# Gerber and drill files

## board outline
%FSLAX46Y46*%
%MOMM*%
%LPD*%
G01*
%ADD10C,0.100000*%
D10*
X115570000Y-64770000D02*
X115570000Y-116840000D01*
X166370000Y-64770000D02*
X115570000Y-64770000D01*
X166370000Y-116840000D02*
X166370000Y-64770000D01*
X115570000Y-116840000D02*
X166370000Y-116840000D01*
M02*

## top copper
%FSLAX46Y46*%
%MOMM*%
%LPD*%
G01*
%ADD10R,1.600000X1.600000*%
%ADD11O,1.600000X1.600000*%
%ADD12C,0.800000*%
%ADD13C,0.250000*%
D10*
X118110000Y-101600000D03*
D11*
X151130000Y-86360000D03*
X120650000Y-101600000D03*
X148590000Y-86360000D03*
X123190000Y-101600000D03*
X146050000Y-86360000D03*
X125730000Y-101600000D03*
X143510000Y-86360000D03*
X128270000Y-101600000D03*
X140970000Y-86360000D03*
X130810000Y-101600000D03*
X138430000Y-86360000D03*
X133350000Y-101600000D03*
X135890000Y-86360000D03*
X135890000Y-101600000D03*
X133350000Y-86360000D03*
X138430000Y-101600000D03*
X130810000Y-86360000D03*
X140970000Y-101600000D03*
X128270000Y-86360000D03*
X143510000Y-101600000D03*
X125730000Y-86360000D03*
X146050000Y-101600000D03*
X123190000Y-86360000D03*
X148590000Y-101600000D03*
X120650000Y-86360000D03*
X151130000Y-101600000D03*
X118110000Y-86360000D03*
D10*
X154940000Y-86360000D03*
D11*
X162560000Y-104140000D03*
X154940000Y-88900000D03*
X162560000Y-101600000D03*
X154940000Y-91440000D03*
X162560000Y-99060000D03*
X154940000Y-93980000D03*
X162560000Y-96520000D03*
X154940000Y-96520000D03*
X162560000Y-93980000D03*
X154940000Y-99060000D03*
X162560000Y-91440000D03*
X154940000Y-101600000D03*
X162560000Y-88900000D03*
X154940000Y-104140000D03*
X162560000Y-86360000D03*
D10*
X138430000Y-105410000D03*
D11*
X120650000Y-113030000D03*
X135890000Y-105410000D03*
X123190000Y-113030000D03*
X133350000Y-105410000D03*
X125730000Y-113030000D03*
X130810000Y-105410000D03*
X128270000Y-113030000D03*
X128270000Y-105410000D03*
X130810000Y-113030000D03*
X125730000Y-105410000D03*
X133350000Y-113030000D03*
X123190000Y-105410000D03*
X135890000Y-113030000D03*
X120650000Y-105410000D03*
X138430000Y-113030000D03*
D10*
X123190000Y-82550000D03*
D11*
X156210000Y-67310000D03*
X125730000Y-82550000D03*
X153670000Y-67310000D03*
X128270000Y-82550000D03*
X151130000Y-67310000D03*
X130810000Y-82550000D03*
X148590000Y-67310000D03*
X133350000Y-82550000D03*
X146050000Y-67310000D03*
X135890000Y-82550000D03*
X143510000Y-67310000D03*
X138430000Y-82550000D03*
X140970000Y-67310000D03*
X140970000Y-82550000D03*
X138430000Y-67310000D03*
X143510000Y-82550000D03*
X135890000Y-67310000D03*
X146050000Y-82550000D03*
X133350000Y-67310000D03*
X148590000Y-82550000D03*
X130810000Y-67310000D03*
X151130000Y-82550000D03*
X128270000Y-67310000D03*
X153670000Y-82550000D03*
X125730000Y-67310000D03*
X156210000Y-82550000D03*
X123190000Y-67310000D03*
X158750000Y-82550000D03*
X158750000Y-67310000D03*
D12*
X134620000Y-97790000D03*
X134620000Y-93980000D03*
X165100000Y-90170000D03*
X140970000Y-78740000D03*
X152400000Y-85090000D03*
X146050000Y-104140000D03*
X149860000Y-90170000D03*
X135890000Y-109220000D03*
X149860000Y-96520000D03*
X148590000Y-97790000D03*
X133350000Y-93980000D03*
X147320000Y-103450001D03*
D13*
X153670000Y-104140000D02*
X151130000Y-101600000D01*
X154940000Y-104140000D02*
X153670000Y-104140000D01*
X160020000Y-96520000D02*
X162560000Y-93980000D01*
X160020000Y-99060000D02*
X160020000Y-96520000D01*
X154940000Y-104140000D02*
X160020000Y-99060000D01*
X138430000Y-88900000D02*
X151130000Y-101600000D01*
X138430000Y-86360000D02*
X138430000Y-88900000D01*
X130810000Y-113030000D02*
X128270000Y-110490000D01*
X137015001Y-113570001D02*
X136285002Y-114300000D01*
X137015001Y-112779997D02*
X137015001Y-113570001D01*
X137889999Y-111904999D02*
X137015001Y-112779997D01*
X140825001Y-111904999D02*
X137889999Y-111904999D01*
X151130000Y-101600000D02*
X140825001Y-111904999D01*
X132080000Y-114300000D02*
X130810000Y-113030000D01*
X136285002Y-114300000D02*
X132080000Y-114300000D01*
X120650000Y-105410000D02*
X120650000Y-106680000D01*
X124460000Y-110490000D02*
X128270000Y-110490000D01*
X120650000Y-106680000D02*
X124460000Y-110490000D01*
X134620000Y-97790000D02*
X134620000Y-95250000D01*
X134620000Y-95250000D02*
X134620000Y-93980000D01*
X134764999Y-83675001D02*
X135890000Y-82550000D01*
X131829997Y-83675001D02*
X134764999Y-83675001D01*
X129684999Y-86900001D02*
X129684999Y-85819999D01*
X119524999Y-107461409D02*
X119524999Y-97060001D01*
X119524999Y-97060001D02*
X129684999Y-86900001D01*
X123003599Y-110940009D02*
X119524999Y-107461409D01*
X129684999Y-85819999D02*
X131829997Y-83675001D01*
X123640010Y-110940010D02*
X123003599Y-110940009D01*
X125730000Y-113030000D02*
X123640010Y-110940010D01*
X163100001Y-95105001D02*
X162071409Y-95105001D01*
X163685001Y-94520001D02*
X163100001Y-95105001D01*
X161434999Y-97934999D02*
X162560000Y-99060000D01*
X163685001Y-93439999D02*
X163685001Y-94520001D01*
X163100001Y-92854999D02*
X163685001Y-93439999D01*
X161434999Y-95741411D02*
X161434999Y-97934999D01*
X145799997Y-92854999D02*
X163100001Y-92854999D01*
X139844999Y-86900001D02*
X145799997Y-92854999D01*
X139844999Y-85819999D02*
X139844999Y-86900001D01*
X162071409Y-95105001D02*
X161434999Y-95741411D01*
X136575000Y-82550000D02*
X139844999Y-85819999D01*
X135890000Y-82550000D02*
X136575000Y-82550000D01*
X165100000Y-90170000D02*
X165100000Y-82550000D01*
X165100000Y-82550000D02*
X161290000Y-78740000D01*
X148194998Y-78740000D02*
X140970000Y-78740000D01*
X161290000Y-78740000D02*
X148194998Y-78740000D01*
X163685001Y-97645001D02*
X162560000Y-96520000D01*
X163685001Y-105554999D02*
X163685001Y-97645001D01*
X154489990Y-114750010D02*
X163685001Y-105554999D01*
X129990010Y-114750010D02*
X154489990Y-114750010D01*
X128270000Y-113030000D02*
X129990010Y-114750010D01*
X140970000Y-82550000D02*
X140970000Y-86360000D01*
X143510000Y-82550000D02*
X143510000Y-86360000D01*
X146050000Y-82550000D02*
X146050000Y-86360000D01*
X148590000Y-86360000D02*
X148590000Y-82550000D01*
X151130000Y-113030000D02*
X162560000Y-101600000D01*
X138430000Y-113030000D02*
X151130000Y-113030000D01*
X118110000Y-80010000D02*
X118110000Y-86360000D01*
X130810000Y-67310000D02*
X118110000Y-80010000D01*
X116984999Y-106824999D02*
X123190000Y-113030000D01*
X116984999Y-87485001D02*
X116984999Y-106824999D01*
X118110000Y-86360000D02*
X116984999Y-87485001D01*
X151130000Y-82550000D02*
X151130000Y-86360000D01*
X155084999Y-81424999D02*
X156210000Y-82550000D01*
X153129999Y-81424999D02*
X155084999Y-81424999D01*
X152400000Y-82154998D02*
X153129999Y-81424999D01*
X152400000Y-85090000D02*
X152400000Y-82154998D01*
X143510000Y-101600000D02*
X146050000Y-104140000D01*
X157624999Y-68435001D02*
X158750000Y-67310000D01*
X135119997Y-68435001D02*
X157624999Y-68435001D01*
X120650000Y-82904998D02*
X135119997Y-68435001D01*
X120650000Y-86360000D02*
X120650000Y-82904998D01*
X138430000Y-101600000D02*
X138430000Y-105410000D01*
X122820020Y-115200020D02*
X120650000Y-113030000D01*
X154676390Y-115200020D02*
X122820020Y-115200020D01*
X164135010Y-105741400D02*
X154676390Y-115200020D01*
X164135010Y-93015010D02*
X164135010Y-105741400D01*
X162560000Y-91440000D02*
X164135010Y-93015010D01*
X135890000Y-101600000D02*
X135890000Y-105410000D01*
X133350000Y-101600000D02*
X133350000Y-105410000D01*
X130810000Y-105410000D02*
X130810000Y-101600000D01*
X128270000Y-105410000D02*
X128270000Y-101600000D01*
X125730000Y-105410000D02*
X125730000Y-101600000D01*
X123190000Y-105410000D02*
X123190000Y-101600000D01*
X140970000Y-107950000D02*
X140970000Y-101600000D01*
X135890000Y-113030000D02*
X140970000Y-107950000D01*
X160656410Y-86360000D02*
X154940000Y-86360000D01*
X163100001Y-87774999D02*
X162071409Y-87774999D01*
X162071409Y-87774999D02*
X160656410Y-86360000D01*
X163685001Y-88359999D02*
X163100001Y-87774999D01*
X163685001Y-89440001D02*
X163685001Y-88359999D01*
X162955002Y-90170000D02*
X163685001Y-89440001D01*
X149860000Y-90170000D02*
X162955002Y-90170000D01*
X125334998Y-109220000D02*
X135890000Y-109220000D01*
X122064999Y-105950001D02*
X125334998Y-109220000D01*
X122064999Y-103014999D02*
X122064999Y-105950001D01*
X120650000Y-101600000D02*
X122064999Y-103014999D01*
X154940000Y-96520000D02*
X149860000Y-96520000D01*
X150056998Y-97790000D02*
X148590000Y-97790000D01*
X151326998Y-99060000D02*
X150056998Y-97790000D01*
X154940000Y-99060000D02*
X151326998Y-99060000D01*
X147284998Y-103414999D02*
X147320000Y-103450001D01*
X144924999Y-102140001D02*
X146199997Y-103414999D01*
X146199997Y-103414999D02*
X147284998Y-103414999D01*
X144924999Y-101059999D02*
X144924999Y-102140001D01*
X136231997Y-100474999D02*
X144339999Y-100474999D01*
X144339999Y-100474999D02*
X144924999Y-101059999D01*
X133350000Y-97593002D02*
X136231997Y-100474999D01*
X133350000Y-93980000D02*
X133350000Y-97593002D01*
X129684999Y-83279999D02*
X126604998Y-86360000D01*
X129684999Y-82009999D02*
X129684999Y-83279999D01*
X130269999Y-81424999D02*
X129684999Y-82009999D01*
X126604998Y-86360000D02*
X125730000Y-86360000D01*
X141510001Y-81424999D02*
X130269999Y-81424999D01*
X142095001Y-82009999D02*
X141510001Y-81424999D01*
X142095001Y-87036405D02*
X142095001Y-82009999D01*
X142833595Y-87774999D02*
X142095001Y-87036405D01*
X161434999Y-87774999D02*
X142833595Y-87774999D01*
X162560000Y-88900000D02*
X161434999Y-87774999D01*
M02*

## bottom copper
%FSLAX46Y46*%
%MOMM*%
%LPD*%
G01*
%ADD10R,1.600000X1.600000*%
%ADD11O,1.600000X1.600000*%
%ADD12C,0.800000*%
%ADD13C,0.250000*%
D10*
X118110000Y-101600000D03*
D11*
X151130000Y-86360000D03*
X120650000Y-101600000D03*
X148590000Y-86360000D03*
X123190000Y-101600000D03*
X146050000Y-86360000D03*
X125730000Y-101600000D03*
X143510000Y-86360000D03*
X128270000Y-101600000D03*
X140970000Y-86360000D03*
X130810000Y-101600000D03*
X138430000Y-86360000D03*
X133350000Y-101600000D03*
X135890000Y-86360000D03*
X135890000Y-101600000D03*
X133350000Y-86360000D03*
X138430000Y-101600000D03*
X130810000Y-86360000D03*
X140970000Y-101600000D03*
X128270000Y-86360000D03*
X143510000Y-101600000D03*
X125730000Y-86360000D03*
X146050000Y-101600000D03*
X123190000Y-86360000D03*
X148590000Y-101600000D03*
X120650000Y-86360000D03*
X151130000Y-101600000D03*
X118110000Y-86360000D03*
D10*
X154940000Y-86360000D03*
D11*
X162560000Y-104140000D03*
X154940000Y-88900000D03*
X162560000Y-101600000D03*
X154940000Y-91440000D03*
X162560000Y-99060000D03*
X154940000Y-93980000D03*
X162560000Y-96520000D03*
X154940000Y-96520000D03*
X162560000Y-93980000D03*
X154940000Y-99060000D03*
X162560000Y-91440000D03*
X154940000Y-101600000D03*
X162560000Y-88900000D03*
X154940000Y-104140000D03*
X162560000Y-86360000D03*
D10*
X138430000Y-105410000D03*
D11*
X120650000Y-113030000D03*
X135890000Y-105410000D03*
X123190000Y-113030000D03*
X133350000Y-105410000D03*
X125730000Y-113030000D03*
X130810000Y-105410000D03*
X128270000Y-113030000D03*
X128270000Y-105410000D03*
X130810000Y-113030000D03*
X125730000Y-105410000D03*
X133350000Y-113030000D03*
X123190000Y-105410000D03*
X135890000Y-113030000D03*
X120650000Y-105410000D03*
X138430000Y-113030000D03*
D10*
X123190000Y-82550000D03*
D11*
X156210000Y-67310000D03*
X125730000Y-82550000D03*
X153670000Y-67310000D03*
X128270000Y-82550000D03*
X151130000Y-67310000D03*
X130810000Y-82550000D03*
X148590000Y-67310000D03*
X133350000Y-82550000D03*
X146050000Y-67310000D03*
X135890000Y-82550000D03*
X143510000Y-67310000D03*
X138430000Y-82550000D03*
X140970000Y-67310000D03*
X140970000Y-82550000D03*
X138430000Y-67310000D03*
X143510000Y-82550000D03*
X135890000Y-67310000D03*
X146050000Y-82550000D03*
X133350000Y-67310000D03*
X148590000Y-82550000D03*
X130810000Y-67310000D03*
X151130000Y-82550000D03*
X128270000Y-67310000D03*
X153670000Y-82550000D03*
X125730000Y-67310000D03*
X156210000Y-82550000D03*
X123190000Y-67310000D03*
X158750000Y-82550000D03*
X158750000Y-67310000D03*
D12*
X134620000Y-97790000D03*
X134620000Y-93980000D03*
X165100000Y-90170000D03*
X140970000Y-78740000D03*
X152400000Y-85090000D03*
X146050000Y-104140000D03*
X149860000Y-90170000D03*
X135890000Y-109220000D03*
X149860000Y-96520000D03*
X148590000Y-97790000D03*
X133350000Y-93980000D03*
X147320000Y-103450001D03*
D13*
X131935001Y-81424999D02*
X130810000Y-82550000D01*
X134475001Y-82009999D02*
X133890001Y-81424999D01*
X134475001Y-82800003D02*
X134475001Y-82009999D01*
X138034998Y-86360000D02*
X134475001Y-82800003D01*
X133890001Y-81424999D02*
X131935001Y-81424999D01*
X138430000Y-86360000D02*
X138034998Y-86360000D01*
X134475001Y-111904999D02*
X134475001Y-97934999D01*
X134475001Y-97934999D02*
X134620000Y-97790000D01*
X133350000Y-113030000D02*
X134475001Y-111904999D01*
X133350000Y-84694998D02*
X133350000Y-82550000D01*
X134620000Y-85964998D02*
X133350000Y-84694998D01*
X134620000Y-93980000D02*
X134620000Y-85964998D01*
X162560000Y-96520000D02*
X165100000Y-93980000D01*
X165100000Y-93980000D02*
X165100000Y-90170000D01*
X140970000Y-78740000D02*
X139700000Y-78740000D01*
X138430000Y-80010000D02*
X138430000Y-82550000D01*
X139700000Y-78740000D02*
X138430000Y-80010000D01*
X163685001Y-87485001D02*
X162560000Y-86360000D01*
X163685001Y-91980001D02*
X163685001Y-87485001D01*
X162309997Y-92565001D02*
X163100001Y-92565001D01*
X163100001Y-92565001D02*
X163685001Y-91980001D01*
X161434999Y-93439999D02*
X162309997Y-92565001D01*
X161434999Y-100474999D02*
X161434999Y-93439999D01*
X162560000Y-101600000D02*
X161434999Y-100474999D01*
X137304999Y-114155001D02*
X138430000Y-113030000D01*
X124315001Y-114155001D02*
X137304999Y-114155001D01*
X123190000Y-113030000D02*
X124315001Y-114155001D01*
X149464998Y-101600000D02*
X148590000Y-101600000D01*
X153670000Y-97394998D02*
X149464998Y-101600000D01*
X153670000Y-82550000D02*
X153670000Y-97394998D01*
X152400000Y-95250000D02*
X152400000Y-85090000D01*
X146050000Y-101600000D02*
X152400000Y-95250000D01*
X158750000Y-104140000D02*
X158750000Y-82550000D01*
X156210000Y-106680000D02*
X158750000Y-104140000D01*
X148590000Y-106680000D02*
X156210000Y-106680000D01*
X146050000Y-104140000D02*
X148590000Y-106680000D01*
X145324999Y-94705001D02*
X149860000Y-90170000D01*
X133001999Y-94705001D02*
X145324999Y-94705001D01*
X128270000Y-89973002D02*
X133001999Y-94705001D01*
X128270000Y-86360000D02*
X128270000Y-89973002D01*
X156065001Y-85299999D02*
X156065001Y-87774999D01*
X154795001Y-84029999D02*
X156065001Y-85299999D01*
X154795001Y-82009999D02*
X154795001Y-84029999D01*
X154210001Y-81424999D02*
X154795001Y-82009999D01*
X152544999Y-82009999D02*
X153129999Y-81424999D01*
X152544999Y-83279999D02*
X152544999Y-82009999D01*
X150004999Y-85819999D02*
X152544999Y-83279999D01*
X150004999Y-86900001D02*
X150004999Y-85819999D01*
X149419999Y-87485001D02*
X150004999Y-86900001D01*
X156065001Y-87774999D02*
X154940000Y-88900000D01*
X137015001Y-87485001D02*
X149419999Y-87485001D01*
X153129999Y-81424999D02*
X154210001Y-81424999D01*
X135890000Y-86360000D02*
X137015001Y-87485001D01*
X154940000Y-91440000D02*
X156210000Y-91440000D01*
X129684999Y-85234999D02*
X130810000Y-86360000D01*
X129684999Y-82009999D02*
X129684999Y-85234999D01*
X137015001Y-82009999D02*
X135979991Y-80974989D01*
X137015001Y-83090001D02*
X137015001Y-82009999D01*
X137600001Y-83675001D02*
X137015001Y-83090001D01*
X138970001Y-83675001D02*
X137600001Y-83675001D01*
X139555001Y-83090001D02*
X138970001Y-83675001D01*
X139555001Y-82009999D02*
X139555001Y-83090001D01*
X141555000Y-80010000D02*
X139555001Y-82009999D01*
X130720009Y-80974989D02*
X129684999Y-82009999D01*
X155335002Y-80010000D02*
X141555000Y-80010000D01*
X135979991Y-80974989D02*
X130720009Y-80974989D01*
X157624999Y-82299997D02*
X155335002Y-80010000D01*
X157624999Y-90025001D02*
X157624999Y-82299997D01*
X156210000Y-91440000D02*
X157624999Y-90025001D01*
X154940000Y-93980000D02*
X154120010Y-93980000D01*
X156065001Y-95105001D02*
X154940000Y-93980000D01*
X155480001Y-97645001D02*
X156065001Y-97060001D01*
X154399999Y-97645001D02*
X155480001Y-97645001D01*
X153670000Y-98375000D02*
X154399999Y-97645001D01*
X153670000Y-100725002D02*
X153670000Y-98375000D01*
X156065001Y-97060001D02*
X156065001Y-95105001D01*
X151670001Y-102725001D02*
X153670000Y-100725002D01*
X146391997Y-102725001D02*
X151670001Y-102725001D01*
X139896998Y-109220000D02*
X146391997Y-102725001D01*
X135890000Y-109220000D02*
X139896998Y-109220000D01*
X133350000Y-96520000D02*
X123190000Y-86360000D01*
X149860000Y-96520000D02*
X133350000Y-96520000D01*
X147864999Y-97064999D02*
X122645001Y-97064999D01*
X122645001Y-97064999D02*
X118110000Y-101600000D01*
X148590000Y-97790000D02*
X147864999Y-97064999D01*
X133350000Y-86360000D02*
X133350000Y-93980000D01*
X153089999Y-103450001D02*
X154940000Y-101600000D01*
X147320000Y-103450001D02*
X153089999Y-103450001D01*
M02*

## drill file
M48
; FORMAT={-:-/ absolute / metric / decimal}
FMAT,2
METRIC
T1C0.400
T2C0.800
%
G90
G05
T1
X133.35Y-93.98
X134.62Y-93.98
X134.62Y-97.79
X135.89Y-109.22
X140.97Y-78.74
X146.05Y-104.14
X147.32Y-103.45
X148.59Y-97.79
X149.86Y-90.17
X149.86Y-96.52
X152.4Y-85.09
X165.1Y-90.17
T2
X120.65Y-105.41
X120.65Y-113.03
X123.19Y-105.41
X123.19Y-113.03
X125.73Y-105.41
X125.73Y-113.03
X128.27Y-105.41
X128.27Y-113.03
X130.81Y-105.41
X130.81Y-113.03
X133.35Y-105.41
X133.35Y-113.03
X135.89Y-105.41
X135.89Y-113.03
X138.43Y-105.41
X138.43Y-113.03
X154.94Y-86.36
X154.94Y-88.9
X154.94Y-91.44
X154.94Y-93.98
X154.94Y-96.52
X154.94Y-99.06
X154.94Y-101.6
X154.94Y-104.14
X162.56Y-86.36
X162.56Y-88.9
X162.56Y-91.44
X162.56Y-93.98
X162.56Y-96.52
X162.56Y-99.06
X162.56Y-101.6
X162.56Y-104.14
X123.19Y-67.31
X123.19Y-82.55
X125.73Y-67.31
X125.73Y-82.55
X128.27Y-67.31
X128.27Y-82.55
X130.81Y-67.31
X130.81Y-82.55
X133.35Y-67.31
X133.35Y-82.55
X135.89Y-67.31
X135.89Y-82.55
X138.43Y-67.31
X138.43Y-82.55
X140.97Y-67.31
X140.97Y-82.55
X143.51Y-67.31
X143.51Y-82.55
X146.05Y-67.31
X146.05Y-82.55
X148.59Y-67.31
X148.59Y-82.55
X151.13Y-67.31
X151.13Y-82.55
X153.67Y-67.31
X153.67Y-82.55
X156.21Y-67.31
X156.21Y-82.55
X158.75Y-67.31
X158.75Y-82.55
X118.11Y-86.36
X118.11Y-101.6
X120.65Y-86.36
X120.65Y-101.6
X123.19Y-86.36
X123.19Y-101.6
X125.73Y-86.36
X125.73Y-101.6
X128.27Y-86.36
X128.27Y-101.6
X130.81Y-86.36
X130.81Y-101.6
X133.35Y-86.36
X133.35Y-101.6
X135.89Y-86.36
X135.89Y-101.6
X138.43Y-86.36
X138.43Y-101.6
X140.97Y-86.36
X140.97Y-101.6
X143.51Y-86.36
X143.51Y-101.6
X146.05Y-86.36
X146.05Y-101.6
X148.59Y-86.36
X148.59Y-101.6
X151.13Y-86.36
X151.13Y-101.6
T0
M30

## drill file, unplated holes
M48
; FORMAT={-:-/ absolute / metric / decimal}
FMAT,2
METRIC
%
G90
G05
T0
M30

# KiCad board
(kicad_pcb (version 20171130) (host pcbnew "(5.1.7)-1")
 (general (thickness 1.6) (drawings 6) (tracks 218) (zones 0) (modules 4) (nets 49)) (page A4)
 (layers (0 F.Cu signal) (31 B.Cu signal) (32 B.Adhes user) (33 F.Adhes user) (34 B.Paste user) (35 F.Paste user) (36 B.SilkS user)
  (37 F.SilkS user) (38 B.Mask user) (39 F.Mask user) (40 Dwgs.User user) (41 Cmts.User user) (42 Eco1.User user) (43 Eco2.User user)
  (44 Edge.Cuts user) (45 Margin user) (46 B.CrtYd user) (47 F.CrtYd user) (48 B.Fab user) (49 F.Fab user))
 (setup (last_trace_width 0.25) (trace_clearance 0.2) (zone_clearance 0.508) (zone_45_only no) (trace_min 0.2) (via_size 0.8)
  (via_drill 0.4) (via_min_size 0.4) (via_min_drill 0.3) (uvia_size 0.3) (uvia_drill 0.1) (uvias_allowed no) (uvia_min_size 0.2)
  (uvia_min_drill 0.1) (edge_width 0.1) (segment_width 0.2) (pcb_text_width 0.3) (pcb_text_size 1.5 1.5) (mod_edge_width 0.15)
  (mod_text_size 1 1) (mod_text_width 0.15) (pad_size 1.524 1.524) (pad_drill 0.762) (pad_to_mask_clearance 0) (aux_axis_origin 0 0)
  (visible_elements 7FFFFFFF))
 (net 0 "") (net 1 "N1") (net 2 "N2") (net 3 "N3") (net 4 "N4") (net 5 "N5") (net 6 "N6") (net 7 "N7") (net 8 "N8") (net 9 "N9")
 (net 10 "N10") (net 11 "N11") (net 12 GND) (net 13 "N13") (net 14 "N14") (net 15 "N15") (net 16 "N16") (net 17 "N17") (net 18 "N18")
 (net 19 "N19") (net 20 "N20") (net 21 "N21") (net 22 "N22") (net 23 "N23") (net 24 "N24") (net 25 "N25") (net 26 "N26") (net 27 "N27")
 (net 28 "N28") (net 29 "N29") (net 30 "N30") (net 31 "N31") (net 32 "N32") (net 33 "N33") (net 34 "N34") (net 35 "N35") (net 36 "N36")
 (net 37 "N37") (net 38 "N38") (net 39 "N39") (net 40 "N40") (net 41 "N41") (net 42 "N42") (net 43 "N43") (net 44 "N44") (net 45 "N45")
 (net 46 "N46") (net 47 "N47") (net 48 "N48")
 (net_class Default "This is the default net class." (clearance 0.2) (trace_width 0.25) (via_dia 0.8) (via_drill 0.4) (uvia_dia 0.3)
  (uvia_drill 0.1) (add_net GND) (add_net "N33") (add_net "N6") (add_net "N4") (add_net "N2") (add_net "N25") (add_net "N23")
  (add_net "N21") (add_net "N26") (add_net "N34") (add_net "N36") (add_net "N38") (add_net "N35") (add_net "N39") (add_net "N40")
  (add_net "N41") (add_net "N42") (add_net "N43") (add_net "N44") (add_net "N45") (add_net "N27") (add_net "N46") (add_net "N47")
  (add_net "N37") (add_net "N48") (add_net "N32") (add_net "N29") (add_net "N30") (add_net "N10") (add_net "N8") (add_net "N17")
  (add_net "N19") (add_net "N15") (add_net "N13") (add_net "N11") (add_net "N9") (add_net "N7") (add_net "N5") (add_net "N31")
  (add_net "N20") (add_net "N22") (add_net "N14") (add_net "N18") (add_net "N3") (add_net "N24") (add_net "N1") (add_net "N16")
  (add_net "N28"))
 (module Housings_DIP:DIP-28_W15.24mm (layer F.Cu) (at 118.11 101.6 90)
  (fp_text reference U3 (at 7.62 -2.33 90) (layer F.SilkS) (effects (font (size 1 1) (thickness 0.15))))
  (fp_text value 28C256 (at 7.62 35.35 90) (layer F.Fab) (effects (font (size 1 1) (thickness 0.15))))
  (pad 1 thru_hole rect (at 0 0 90) (size 1.6 1.6) (drill 0.8) (layers *.Cu *.Mask) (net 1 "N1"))
  (pad 15 thru_hole oval (at 15.24 33.02 90) (size 1.6 1.6) (drill 0.8) (layers *.Cu *.Mask) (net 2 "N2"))
  (pad 2 thru_hole oval (at 0 2.54 90) (size 1.6 1.6) (drill 0.8) (layers *.Cu *.Mask) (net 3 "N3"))
  (pad 16 thru_hole oval (at 15.24 30.48 90) (size 1.6 1.6) (drill 0.8) (layers *.Cu *.Mask) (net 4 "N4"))
  (pad 3 thru_hole oval (at 0 5.08 90) (size 1.6 1.6) (drill 0.8) (layers *.Cu *.Mask) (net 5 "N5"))
  (pad 17 thru_hole oval (at 15.24 27.94 90) (size 1.6 1.6) (drill 0.8) (layers *.Cu *.Mask) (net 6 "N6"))
  (pad 4 thru_hole oval (at 0 7.62 90) (size 1.6 1.6) (drill 0.8) (layers *.Cu *.Mask) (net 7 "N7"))
  (pad 18 thru_hole oval (at 15.24 25.4 90) (size 1.6 1.6) (drill 0.8) (layers *.Cu *.Mask) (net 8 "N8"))
  (pad 5 thru_hole oval (at 0 10.16 90) (size 1.6 1.6) (drill 0.8) (layers *.Cu *.Mask) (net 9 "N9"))
  (pad 19 thru_hole oval (at 15.24 22.86 90) (size 1.6 1.6) (drill 0.8) (layers *.Cu *.Mask) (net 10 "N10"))
  (pad 6 thru_hole oval (at 0 12.7 90) (size 1.6 1.6) (drill 0.8) (layers *.Cu *.Mask) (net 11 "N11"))
  (pad 20 thru_hole oval (at 15.24 20.32 90) (size 1.6 1.6) (drill 0.8) (layers *.Cu *.Mask) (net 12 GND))
  (pad 7 thru_hole oval (at 0 15.24 90) (size 1.6 1.6) (drill 0.8) (layers *.Cu *.Mask) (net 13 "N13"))
  (pad 21 thru_hole oval (at 15.24 17.78 90) (size 1.6 1.6) (drill 0.8) (layers *.Cu *.Mask) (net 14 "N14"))
  (pad 8 thru_hole oval (at 0 17.78 90) (size 1.6 1.6) (drill 0.8) (layers *.Cu *.Mask) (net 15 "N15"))
  (pad 22 thru_hole oval (at 15.24 15.24 90) (size 1.6 1.6) (drill 0.8) (layers *.Cu *.Mask) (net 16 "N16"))
  (pad 9 thru_hole oval (at 0 20.32 90) (size 1.6 1.6) (drill 0.8) (layers *.Cu *.Mask) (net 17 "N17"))
  (pad 23 thru_hole oval (at 15.24 12.7 90) (size 1.6 1.6) (drill 0.8) (layers *.Cu *.Mask) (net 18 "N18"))
  (pad 10 thru_hole oval (at 0 22.86 90) (size 1.6 1.6) (drill 0.8) (layers *.Cu *.Mask) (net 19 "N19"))
  (pad 24 thru_hole oval (at 15.24 10.16 90) (size 1.6 1.6) (drill 0.8) (layers *.Cu *.Mask) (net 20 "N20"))
  (pad 11 thru_hole oval (at 0 25.4 90) (size 1.6 1.6) (drill 0.8) (layers *.Cu *.Mask) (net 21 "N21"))
  (pad 25 thru_hole oval (at 15.24 7.62 90) (size 1.6 1.6) (drill 0.8) (layers *.Cu *.Mask) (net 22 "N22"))
  (pad 12 thru_hole oval (at 0 27.94 90) (size 1.6 1.6) (drill 0.8) (layers *.Cu *.Mask) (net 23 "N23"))
  (pad 26 thru_hole oval (at 15.24 5.08 90) (size 1.6 1.6) (drill 0.8) (layers *.Cu *.Mask) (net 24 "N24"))
  (pad 13 thru_hole oval (at 0 30.48 90) (size 1.6 1.6) (drill 0.8) (layers *.Cu *.Mask) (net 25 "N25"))
  (pad 27 thru_hole oval (at 15.24 2.54 90) (size 1.6 1.6) (drill 0.8) (layers *.Cu *.Mask) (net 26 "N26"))
  (pad 14 thru_hole oval (at 0 33.02 90) (size 1.6 1.6) (drill 0.8) (layers *.Cu *.Mask) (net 12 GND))
  (pad 28 thru_hole oval (at 15.24 0 90) (size 1.6 1.6) (drill 0.8) (layers *.Cu *.Mask) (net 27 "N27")))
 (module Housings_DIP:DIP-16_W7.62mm (layer F.Cu) (at 154.94 86.36)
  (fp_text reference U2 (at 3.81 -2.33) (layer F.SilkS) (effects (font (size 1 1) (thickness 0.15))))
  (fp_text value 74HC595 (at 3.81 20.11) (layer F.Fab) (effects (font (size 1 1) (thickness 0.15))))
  (pad 1 thru_hole rect (at 0 0) (size 1.6 1.6) (drill 0.8) (layers *.Cu *.Mask) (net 20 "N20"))
  (pad 9 thru_hole oval (at 7.62 17.78) (size 1.6 1.6) (drill 0.8) (layers *.Cu *.Mask) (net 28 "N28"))
  (pad 2 thru_hole oval (at 0 2.54) (size 1.6 1.6) (drill 0.8) (layers *.Cu *.Mask) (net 14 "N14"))
  (pad 10 thru_hole oval (at 7.62 15.24) (size 1.6 1.6) (drill 0.8) (layers *.Cu *.Mask) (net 27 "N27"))
  (pad 3 thru_hole oval (at 0 5.08) (size 1.6 1.6) (drill 0.8) (layers *.Cu *.Mask) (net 18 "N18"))
  (pad 11 thru_hole oval (at 7.62 12.7) (size 1.6 1.6) (drill 0.8) (layers *.Cu *.Mask) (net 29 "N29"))
  (pad 4 thru_hole oval (at 0 7.62) (size 1.6 1.6) (drill 0.8) (layers *.Cu *.Mask) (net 3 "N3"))
  (pad 12 thru_hole oval (at 7.62 10.16) (size 1.6 1.6) (drill 0.8) (layers *.Cu *.Mask) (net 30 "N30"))
  (pad 5 thru_hole oval (at 0 10.16) (size 1.6 1.6) (drill 0.8) (layers *.Cu *.Mask) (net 24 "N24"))
  (pad 13 thru_hole oval (at 7.62 7.62) (size 1.6 1.6) (drill 0.8) (layers *.Cu *.Mask) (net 12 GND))
  (pad 6 thru_hole oval (at 0 12.7) (size 1.6 1.6) (drill 0.8) (layers *.Cu *.Mask) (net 1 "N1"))
  (pad 14 thru_hole oval (at 7.62 5.08) (size 1.6 1.6) (drill 0.8) (layers *.Cu *.Mask) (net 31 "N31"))
  (pad 7 thru_hole oval (at 0 15.24) (size 1.6 1.6) (drill 0.8) (layers *.Cu *.Mask) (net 16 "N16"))
  (pad 15 thru_hole oval (at 7.62 2.54) (size 1.6 1.6) (drill 0.8) (layers *.Cu *.Mask) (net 22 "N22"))
  (pad 8 thru_hole oval (at 0 17.78) (size 1.6 1.6) (drill 0.8) (layers *.Cu *.Mask) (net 12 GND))
  (pad 16 thru_hole oval (at 7.62 0) (size 1.6 1.6) (drill 0.8) (layers *.Cu *.Mask) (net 27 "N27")))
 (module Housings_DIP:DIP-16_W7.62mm (layer F.Cu) (at 138.43 105.41 270)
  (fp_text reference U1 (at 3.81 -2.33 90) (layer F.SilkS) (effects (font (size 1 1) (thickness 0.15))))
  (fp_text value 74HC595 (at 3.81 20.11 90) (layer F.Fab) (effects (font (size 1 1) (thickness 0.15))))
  (pad 1 thru_hole rect (at 0 0 270) (size 1.6 1.6) (drill 0.8) (layers *.Cu *.Mask) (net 17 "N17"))
  (pad 9 thru_hole oval (at 7.62 17.78 270) (size 1.6 1.6) (drill 0.8) (layers *.Cu *.Mask) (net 31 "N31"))
  (pad 2 thru_hole oval (at 0 2.54 270) (size 1.6 1.6) (drill 0.8) (layers *.Cu *.Mask) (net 15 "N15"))
  (pad 10 thru_hole oval (at 7.62 15.24 270) (size 1.6 1.6) (drill 0.8) (layers *.Cu *.Mask) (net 27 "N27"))
  (pad 3 thru_hole oval (at 0 5.08 270) (size 1.6 1.6) (drill 0.8) (layers *.Cu *.Mask) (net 13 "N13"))
  (pad 11 thru_hole oval (at 7.62 12.7 270) (size 1.6 1.6) (drill 0.8) (layers *.Cu *.Mask) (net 29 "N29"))
  (pad 4 thru_hole oval (at 0 7.62 270) (size 1.6 1.6) (drill 0.8) (layers *.Cu *.Mask) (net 11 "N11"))
  (pad 12 thru_hole oval (at 7.62 10.16 270) (size 1.6 1.6) (drill 0.8) (layers *.Cu *.Mask) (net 30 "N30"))
  (pad 5 thru_hole oval (at 0 10.16 270) (size 1.6 1.6) (drill 0.8) (layers *.Cu *.Mask) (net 9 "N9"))
  (pad 13 thru_hole oval (at 7.62 7.62 270) (size 1.6 1.6) (drill 0.8) (layers *.Cu *.Mask) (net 12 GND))
  (pad 6 thru_hole oval (at 0 12.7 270) (size 1.6 1.6) (drill 0.8) (layers *.Cu *.Mask) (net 7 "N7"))
  (pad 14 thru_hole oval (at 7.62 5.08 270) (size 1.6 1.6) (drill 0.8) (layers *.Cu *.Mask) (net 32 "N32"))
  (pad 7 thru_hole oval (at 0 15.24 270) (size 1.6 1.6) (drill 0.8) (layers *.Cu *.Mask) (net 5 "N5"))
  (pad 15 thru_hole oval (at 7.62 2.54 270) (size 1.6 1.6) (drill 0.8) (layers *.Cu *.Mask) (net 19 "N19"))
  (pad 8 thru_hole oval (at 0 17.78 270) (size 1.6 1.6) (drill 0.8) (layers *.Cu *.Mask) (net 12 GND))
  (pad 16 thru_hole oval (at 7.62 0 270) (size 1.6 1.6) (drill 0.8) (layers *.Cu *.Mask) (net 27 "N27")))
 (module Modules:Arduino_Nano (layer F.Cu) (at 123.19 82.55 90)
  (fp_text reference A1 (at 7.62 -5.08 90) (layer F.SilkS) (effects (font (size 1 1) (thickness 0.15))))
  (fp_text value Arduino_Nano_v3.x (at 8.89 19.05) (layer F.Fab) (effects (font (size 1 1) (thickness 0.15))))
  (pad 1 thru_hole rect (at 0 0 90) (size 1.6 1.6) (drill 0.8) (layers *.Cu *.Mask) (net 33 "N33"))
  (pad 17 thru_hole oval (at 15.24 33.02 90) (size 1.6 1.6) (drill 0.8) (layers *.Cu *.Mask) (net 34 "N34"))
  (pad 2 thru_hole oval (at 0 2.54 90) (size 1.6 1.6) (drill 0.8) (layers *.Cu *.Mask) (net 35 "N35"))
  (pad 18 thru_hole oval (at 15.24 30.48 90) (size 1.6 1.6) (drill 0.8) (layers *.Cu *.Mask) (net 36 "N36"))
  (pad 3 thru_hole oval (at 0 5.08 90) (size 1.6 1.6) (drill 0.8) (layers *.Cu *.Mask) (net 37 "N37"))
  (pad 19 thru_hole oval (at 15.24 27.94 90) (size 1.6 1.6) (drill 0.8) (layers *.Cu *.Mask) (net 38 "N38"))
  (pad 4 thru_hole oval (at 0 7.62 90) (size 1.6 1.6) (drill 0.8) (layers *.Cu *.Mask) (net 12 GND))
  (pad 20 thru_hole oval (at 15.24 25.4 90) (size 1.6 1.6) (drill 0.8) (layers *.Cu *.Mask) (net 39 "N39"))
  (pad 5 thru_hole oval (at 0 10.16 90) (size 1.6 1.6) (drill 0.8) (layers *.Cu *.Mask) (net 32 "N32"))
  (pad 21 thru_hole oval (at 15.24 22.86 90) (size 1.6 1.6) (drill 0.8) (layers *.Cu *.Mask) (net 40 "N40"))
  (pad 6 thru_hole oval (at 0 12.7 90) (size 1.6 1.6) (drill 0.8) (layers *.Cu *.Mask) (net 29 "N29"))
  (pad 22 thru_hole oval (at 15.24 20.32 90) (size 1.6 1.6) (drill 0.8) (layers *.Cu *.Mask) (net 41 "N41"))
  (pad 7 thru_hole oval (at 0 15.24 90) (size 1.6 1.6) (drill 0.8) (layers *.Cu *.Mask) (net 30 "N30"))
  (pad 23 thru_hole oval (at 15.24 17.78 90) (size 1.6 1.6) (drill 0.8) (layers *.Cu *.Mask) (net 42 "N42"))
  (pad 8 thru_hole oval (at 0 17.78 90) (size 1.6 1.6) (drill 0.8) (layers *.Cu *.Mask) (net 10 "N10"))
  (pad 24 thru_hole oval (at 15.24 15.24 90) (size 1.6 1.6) (drill 0.8) (layers *.Cu *.Mask) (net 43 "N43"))
  (pad 9 thru_hole oval (at 0 20.32 90) (size 1.6 1.6) (drill 0.8) (layers *.Cu *.Mask) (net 8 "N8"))
  (pad 25 thru_hole oval (at 15.24 12.7 90) (size 1.6 1.6) (drill 0.8) (layers *.Cu *.Mask) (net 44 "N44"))
  (pad 10 thru_hole oval (at 0 22.86 90) (size 1.6 1.6) (drill 0.8) (layers *.Cu *.Mask) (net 6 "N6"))
  (pad 26 thru_hole oval (at 15.24 10.16 90) (size 1.6 1.6) (drill 0.8) (layers *.Cu *.Mask) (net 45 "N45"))
  (pad 11 thru_hole oval (at 0 25.4 90) (size 1.6 1.6) (drill 0.8) (layers *.Cu *.Mask) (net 4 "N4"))
  (pad 27 thru_hole oval (at 15.24 7.62 90) (size 1.6 1.6) (drill 0.8) (layers *.Cu *.Mask) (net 27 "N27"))
  (pad 12 thru_hole oval (at 0 27.94 90) (size 1.6 1.6) (drill 0.8) (layers *.Cu *.Mask) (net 2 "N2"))
  (pad 28 thru_hole oval (at 15.24 5.08 90) (size 1.6 1.6) (drill 0.8) (layers *.Cu *.Mask) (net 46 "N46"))
  (pad 13 thru_hole oval (at 0 30.48 90) (size 1.6 1.6) (drill 0.8) (layers *.Cu *.Mask) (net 25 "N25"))
  (pad 29 thru_hole oval (at 15.24 2.54 90) (size 1.6 1.6) (drill 0.8) (layers *.Cu *.Mask) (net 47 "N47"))
  (pad 14 thru_hole oval (at 0 33.02 90) (size 1.6 1.6) (drill 0.8) (layers *.Cu *.Mask) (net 23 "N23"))
  (pad 30 thru_hole oval (at 15.24 0 90) (size 1.6 1.6) (drill 0.8) (layers *.Cu *.Mask) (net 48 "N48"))
  (pad 15 thru_hole oval (at 0 35.56 90) (size 1.6 1.6) (drill 0.8) (layers *.Cu *.Mask) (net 21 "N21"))
  (pad 16 thru_hole oval (at 15.24 35.56 90) (size 1.6 1.6) (drill 0.8) (layers *.Cu *.Mask) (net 26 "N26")))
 (gr_line (start 115.57 64.77) (end 115.57 116.84) (layer Edge.Cuts) (width 0.1))
 (gr_line (start 166.37 64.77) (end 115.57 64.77) (layer Edge.Cuts) (width 0.1))
 (gr_line (start 166.37 116.84) (end 166.37 64.77) (layer Edge.Cuts) (width 0.1))
 (gr_line (start 115.57 116.84) (end 166.37 116.84) (layer Edge.Cuts) (width 0.1))
 (segment (start 153.67 104.14) (end 151.13 101.6) (width 0.25) (layer F.Cu) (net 12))
 (segment (start 154.94 104.14) (end 153.67 104.14) (width 0.25) (layer F.Cu) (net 12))
 (segment (start 160.02 96.52) (end 162.56 93.98) (width 0.25) (layer F.Cu) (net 12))
 (segment (start 160.02 99.06) (end 160.02 96.52) (width 0.25) (layer F.Cu) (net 12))
 (segment (start 154.94 104.14) (end 160.02 99.06) (width 0.25) (layer F.Cu) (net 12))
 (segment (start 138.43 88.9) (end 151.13 101.6) (width 0.25) (layer F.Cu) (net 12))
 (segment (start 138.43 86.36) (end 138.43 88.9) (width 0.25) (layer F.Cu) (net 12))
 (segment (start 130.81 113.03) (end 128.27 110.49) (width 0.25) (layer F.Cu) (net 12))
 (segment (start 137.015001 113.570001) (end 136.285002 114.3) (width 0.25) (layer F.Cu) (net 12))
 (segment (start 137.015001 112.779997) (end 137.015001 113.570001) (width 0.25) (layer F.Cu) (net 12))
 (segment (start 137.889999 111.904999) (end 137.015001 112.779997) (width 0.25) (layer F.Cu) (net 12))
 (segment (start 140.825001 111.904999) (end 137.889999 111.904999) (width 0.25) (layer F.Cu) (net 12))
 (segment (start 151.13 101.6) (end 140.825001 111.904999) (width 0.25) (layer F.Cu) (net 12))
 (segment (start 132.08 114.3) (end 130.81 113.03) (width 0.25) (layer F.Cu) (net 12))
 (segment (start 136.285002 114.3) (end 132.08 114.3) (width 0.25) (layer F.Cu) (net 12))
 (segment (start 131.935001 81.424999) (end 130.81 82.55) (width 0.25) (layer B.Cu) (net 12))
 (segment (start 134.475001 82.009999) (end 133.890001 81.424999) (width 0.25) (layer B.Cu) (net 12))
 (segment (start 134.475001 82.800003) (end 134.475001 82.009999) (width 0.25) (layer B.Cu) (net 12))
 (segment (start 138.034998 86.36) (end 134.475001 82.800003) (width 0.25) (layer B.Cu) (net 12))
 (segment (start 133.890001 81.424999) (end 131.935001 81.424999) (width 0.25) (layer B.Cu) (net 12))
 (segment (start 138.43 86.36) (end 138.034998 86.36) (width 0.25) (layer B.Cu) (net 12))
 (segment (start 120.65 105.41) (end 120.65 106.68) (width 0.25) (layer F.Cu) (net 12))
 (segment (start 124.46 110.49) (end 128.27 110.49) (width 0.25) (layer F.Cu) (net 12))
 (segment (start 120.65 106.68) (end 124.46 110.49) (width 0.25) (layer F.Cu) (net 12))
 (segment (start 134.475001 111.904999) (end 134.475001 97.934999) (width 0.25) (layer B.Cu) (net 32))
 (via (at 134.62 97.79) (size 0.8) (drill 0.4) (layers F.Cu B.Cu) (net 32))
 (segment (start 134.475001 97.934999) (end 134.62 97.79) (width 0.25) (layer B.Cu) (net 32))
 (segment (start 133.35 113.03) (end 134.475001 111.904999) (width 0.25) (layer B.Cu) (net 32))
 (segment (start 134.62 97.79) (end 134.62 95.25) (width 0.25) (layer F.Cu) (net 32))
 (via (at 134.62 93.98) (size 0.8) (drill 0.4) (layers F.Cu B.Cu) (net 32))
 (segment (start 134.62 95.25) (end 134.62 93.98) (width 0.25) (layer F.Cu) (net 32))
 (segment (start 133.35 84.694998) (end 133.35 82.55) (width 0.25) (layer B.Cu) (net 32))
 (segment (start 134.62 85.964998) (end 133.35 84.694998) (width 0.25) (layer B.Cu) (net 32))
 (segment (start 134.62 93.98) (end 134.62 85.964998) (width 0.25) (layer B.Cu) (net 32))
 (segment (start 134.764999 83.675001) (end 135.89 82.55) (width 0.25) (layer F.Cu) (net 29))
 (segment (start 131.829997 83.675001) (end 134.764999 83.675001) (width 0.25) (layer F.Cu) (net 29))
 (segment (start 129.684999 86.900001) (end 129.684999 85.819999) (width 0.25) (layer F.Cu) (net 29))
 (segment (start 119.524999 107.461409) (end 119.524999 97.060001) (width 0.25) (layer F.Cu) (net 29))
 (segment (start 119.524999 97.060001) (end 129.684999 86.900001) (width 0.25) (layer F.Cu) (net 29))
 (segment (start 123.003599 110.940009) (end 119.524999 107.461409) (width 0.25) (layer F.Cu) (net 29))
 (segment (start 129.684999 85.819999) (end 131.829997 83.675001) (width 0.25) (layer F.Cu) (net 29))
 (segment (start 123.64001 110.94001) (end 123.003599 110.940009) (width 0.25) (layer F.Cu) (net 29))
 (segment (start 125.73 113.03) (end 123.64001 110.94001) (width 0.25) (layer F.Cu) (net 29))
 (segment (start 163.100001 95.105001) (end 162.071409 95.105001) (width 0.25) (layer F.Cu) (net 29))
 (segment (start 163.685001 94.520001) (end 163.100001 95.105001) (width 0.25) (layer F.Cu) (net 29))
 (segment (start 161.434999 97.934999) (end 162.56 99.06) (width 0.25) (layer F.Cu) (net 29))
 (segment (start 163.685001 93.439999) (end 163.685001 94.520001) (width 0.25) (layer F.Cu) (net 29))
 (segment (start 163.100001 92.854999) (end 163.685001 93.439999) (width 0.25) (layer F.Cu) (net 29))
 (segment (start 161.434999 95.741411) (end 161.434999 97.934999) (width 0.25) (layer F.Cu) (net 29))
 (segment (start 145.799997 92.854999) (end 163.100001 92.854999) (width 0.25) (layer F.Cu) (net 29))
 (segment (start 139.844999 86.900001) (end 145.799997 92.854999) (width 0.25) (layer F.Cu) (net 29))
 (segment (start 139.844999 85.819999) (end 139.844999 86.900001) (width 0.25) (layer F.Cu) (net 29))
 (segment (start 162.071409 95.105001) (end 161.434999 95.741411) (width 0.25) (layer F.Cu) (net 29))
 (segment (start 136.575 82.55) (end 139.844999 85.819999) (width 0.25) (layer F.Cu) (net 29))
 (segment (start 135.89 82.55) (end 136.575 82.55) (width 0.25) (layer F.Cu) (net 29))
 (segment (start 162.56 96.52) (end 165.1 93.98) (width 0.25) (layer B.Cu) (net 30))
 (via (at 165.1 90.17) (size 0.8) (drill 0.4) (layers F.Cu B.Cu) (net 30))
 (segment (start 165.1 93.98) (end 165.1 90.17) (width 0.25) (layer B.Cu) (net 30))
 (segment (start 165.1 90.17) (end 165.1 82.55) (width 0.25) (layer F.Cu) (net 30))
 (segment (start 165.1 82.55) (end 161.29 78.74) (width 0.25) (layer F.Cu) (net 30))
 (via (at 140.97 78.74) (size 0.8) (drill 0.4) (layers F.Cu B.Cu) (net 30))
 (segment (start 148.194998 78.74) (end 140.97 78.74) (width 0.25) (layer F.Cu) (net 30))
 (segment (start 161.29 78.74) (end 148.194998 78.74) (width 0.25) (layer F.Cu) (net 30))
 (segment (start 140.97 78.74) (end 139.7 78.74) (width 0.25) (layer B.Cu) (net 30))
 (segment (start 138.43 80.01) (end 138.43 82.55) (width 0.25) (layer B.Cu) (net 30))
 (segment (start 139.7 78.74) (end 138.43 80.01) (width 0.25) (layer B.Cu) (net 30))
 (segment (start 163.685001 97.645001) (end 162.56 96.52) (width 0.25) (layer F.Cu) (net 30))
 (segment (start 163.685001 105.554999) (end 163.685001 97.645001) (width 0.25) (layer F.Cu) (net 30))
 (segment (start 154.48999 114.75001) (end 163.685001 105.554999) (width 0.25) (layer F.Cu) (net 30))
 (segment (start 129.99001 114.75001) (end 154.48999 114.75001) (width 0.25) (layer F.Cu) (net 30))
 (segment (start 128.27 113.03) (end 129.99001 114.75001) (width 0.25) (layer F.Cu) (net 30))
 (segment (start 140.97 82.55) (end 140.97 86.36) (width 0.25) (layer F.Cu) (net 10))
 (segment (start 143.51 82.55) (end 143.51 86.36) (width 0.25) (layer F.Cu) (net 8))
 (segment (start 146.05 82.55) (end 146.05 86.36) (width 0.25) (layer F.Cu) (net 6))
 (segment (start 148.59 86.36) (end 148.59 82.55) (width 0.25) (layer F.Cu) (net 4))
 (segment (start 163.685001 87.485001) (end 162.56 86.36) (width 0.25) (layer B.Cu) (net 27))
 (segment (start 163.685001 91.980001) (end 163.685001 87.485001) (width 0.25) (layer B.Cu) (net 27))
 (segment (start 162.309997 92.565001) (end 163.100001 92.565001) (width 0.25) (layer B.Cu) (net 27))
 (segment (start 163.100001 92.565001) (end 163.685001 91.980001) (width 0.25) (layer B.Cu) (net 27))
 (segment (start 161.434999 93.439999) (end 162.309997 92.565001) (width 0.25) (layer B.Cu) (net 27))
 (segment (start 161.434999 100.474999) (end 161.434999 93.439999) (width 0.25) (layer B.Cu) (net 27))
 (segment (start 162.56 101.6) (end 161.434999 100.474999) (width 0.25) (layer B.Cu) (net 27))
 (segment (start 137.304999 114.155001) (end 138.43 113.03) (width 0.25) (layer B.Cu) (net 27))
 (segment (start 124.315001 114.155001) (end 137.304999 114.155001) (width 0.25) (layer B.Cu) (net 27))
 (segment (start 123.19 113.03) (end 124.315001 114.155001) (width 0.25) (layer B.Cu) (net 27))
 (segment (start 151.13 113.03) (end 162.56 101.6) (width 0.25) (layer F.Cu) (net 27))
 (segment (start 138.43 113.03) (end 151.13 113.03) (width 0.25) (layer F.Cu) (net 27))
 (segment (start 118.11 80.01) (end 118.11 86.36) (width 0.25) (layer F.Cu) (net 27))
 (segment (start 130.81 67.31) (end 118.11 80.01) (width 0.25) (layer F.Cu) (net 27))
 (segment (start 116.984999 106.824999) (end 123.19 113.03) (width 0.25) (layer F.Cu) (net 27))
 (segment (start 116.984999 87.485001) (end 116.984999 106.824999) (width 0.25) (layer F.Cu) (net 27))
 (segment (start 118.11 86.36) (end 116.984999 87.485001) (width 0.25) (layer F.Cu) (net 27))
 (segment (start 151.13 82.55) (end 151.13 86.36) (width 0.25) (layer F.Cu) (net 2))
 (segment (start 149.464998 101.6) (end 148.59 101.6) (width 0.25) (layer B.Cu) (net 25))
 (segment (start 153.67 97.394998) (end 149.464998 101.6) (width 0.25) (layer B.Cu) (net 25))
 (segment (start 153.67 82.55) (end 153.67 97.394998) (width 0.25) (layer B.Cu) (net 25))
 (via (at 152.4 85.09) (size 0.8) (drill 0.4) (layers F.Cu B.Cu) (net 23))
 (segment (start 152.4 95.25) (end 152.4 85.09) (width 0.25) (layer B.Cu) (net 23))
 (segment (start 146.05 101.6) (end 152.4 95.25) (width 0.25) (layer B.Cu) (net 23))
 (segment (start 155.084999 81.424999) (end 156.21 82.55) (width 0.25) (layer F.Cu) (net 23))
 (segment (start 153.129999 81.424999) (end 155.084999 81.424999) (width 0.25) (layer F.Cu) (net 23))
 (segment (start 152.4 82.154998) (end 153.129999 81.424999) (width 0.25) (layer F.Cu) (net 23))
 (segment (start 152.4 85.09) (end 152.4 82.154998) (width 0.25) (layer F.Cu) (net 23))
 (via (at 146.05 104.14) (size 0.8) (drill 0.4) (layers F.Cu B.Cu) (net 21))
 (segment (start 143.51 101.6) (end 146.05 104.14) (width 0.25) (layer F.Cu) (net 21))
 (segment (start 158.75 104.14) (end 158.75 82.55) (width 0.25) (layer B.Cu) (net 21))
 (segment (start 156.21 106.68) (end 158.75 104.14) (width 0.25) (layer B.Cu) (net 21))
 (segment (start 148.59 106.68) (end 156.21 106.68) (width 0.25) (layer B.Cu) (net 21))
 (segment (start 146.05 104.14) (end 148.59 106.68) (width 0.25) (layer B.Cu) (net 21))
 (segment (start 157.624999 68.435001) (end 158.75 67.31) (width 0.25) (layer F.Cu) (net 26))
 (segment (start 135.119997 68.435001) (end 157.624999 68.435001) (width 0.25) (layer F.Cu) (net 26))
 (segment (start 120.65 82.904998) (end 135.119997 68.435001) (width 0.25) (layer F.Cu) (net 26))
 (segment (start 120.65 86.36) (end 120.65 82.904998) (width 0.25) (layer F.Cu) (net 26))
 (segment (start 138.43 101.6) (end 138.43 105.41) (width 0.25) (layer F.Cu) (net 17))
 (segment (start 122.82002 115.20002) (end 120.65 113.03) (width 0.25) (layer F.Cu) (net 31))
 (segment (start 154.67639 115.20002) (end 122.82002 115.20002) (width 0.25) (layer F.Cu) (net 31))
 (segment (start 164.13501 105.7414) (end 154.67639 115.20002) (width 0.25) (layer F.Cu) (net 31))
 (segment (start 164.13501 93.01501) (end 164.13501 105.7414) (width 0.25) (layer F.Cu) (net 31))
 (segment (start 162.56 91.44) (end 164.13501 93.01501) (width 0.25) (layer F.Cu) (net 31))
 (segment (start 135.89 101.6) (end 135.89 105.41) (width 0.25) (layer F.Cu) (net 15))
 (segment (start 133.35 101.6) (end 133.35 105.41) (width 0.25) (layer F.Cu) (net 13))
 (segment (start 130.81 105.41) (end 130.81 101.6) (width 0.25) (layer F.Cu) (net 11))
 (segment (start 128.27 105.41) (end 128.27 101.6) (width 0.25) (layer F.Cu) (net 9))
 (segment (start 125.73 105.41) (end 125.73 101.6) (width 0.25) (layer F.Cu) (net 7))
 (segment (start 123.19 105.41) (end 123.19 101.6) (width 0.25) (layer F.Cu) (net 5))
 (segment (start 140.97 107.95) (end 140.97 101.6) (width 0.25) (layer F.Cu) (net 19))
 (segment (start 135.89 113.03) (end 140.97 107.95) (width 0.25) (layer F.Cu) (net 19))
 (via (at 149.86 90.17) (size 0.8) (drill 0.4) (layers F.Cu B.Cu) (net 20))
 (segment (start 145.324999 94.705001) (end 149.86 90.17) (width 0.25) (layer B.Cu) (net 20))
 (segment (start 133.001999 94.705001) (end 145.324999 94.705001) (width 0.25) (layer B.Cu) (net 20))
 (segment (start 128.27 89.973002) (end 133.001999 94.705001) (width 0.25) (layer B.Cu) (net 20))
 (segment (start 128.27 86.36) (end 128.27 89.973002) (width 0.25) (layer B.Cu) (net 20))
 (segment (start 160.65641 86.36) (end 154.94 86.36) (width 0.25) (layer F.Cu) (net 20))
 (segment (start 163.100001 87.774999) (end 162.071409 87.774999) (width 0.25) (layer F.Cu) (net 20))
 (segment (start 162.071409 87.774999) (end 160.65641 86.36) (width 0.25) (layer F.Cu) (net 20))
 (segment (start 163.685001 88.359999) (end 163.100001 87.774999) (width 0.25) (layer F.Cu) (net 20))
 (segment (start 163.685001 89.440001) (end 163.685001 88.359999) (width 0.25) (layer F.Cu) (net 20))
 (segment (start 162.955002 90.17) (end 163.685001 89.440001) (width 0.25) (layer F.Cu) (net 20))
 (segment (start 149.86 90.17) (end 162.955002 90.17) (width 0.25) (layer F.Cu) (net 20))
 (segment (start 156.065001 85.299999) (end 156.065001 87.774999) (width 0.25) (layer B.Cu) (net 14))
 (segment (start 154.795001 84.029999) (end 156.065001 85.299999) (width 0.25) (layer B.Cu) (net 14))
 (segment (start 154.795001 82.009999) (end 154.795001 84.029999) (width 0.25) (layer B.Cu) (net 14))
 (segment (start 154.210001 81.424999) (end 154.795001 82.009999) (width 0.25) (layer B.Cu) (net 14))
 (segment (start 152.544999 82.009999) (end 153.129999 81.424999) (width 0.25) (layer B.Cu) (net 14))
 (segment (start 152.544999 83.279999) (end 152.544999 82.009999) (width 0.25) (layer B.Cu) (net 14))
 (segment (start 150.004999 85.819999) (end 152.544999 83.279999) (width 0.25) (layer B.Cu) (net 14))
 (segment (start 150.004999 86.900001) (end 150.004999 85.819999) (width 0.25) (layer B.Cu) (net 14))
 (segment (start 149.419999 87.485001) (end 150.004999 86.900001) (width 0.25) (layer B.Cu) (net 14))
 (segment (start 156.065001 87.774999) (end 154.94 88.9) (width 0.25) (layer B.Cu) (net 14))
 (segment (start 137.015001 87.485001) (end 149.419999 87.485001) (width 0.25) (layer B.Cu) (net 14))
 (segment (start 153.129999 81.424999) (end 154.210001 81.424999) (width 0.25) (layer B.Cu) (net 14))
 (segment (start 135.89 86.36) (end 137.015001 87.485001) (width 0.25) (layer B.Cu) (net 14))
 (segment (start 154.94 91.44) (end 156.21 91.44) (width 0.25) (layer B.Cu) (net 18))
 (segment (start 129.684999 85.234999) (end 130.81 86.36) (width 0.25) (layer B.Cu) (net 18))
 (segment (start 129.684999 82.009999) (end 129.684999 85.234999) (width 0.25) (layer B.Cu) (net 18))
 (segment (start 137.015001 82.009999) (end 135.979991 80.974989) (width 0.25) (layer B.Cu) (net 18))
 (segment (start 137.015001 83.090001) (end 137.015001 82.009999) (width 0.25) (layer B.Cu) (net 18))
 (segment (start 137.600001 83.675001) (end 137.015001 83.090001) (width 0.25) (layer B.Cu) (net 18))
 (segment (start 138.970001 83.675001) (end 137.600001 83.675001) (width 0.25) (layer B.Cu) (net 18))
 (segment (start 139.555001 83.090001) (end 138.970001 83.675001) (width 0.25) (layer B.Cu) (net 18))
 (segment (start 139.555001 82.009999) (end 139.555001 83.090001) (width 0.25) (layer B.Cu) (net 18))
 (segment (start 141.555 80.01) (end 139.555001 82.009999) (width 0.25) (layer B.Cu) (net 18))
 (segment (start 130.720009 80.974989) (end 129.684999 82.009999) (width 0.25) (layer B.Cu) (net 18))
 (segment (start 155.335002 80.01) (end 141.555 80.01) (width 0.25) (layer B.Cu) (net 18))
 (segment (start 135.979991 80.974989) (end 130.720009 80.974989) (width 0.25) (layer B.Cu) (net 18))
 (segment (start 157.624999 82.299997) (end 155.335002 80.01) (width 0.25) (layer B.Cu) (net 18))
 (segment (start 157.624999 90.025001) (end 157.624999 82.299997) (width 0.25) (layer B.Cu) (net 18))
 (segment (start 156.21 91.44) (end 157.624999 90.025001) (width 0.25) (layer B.Cu) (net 18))
 (segment (start 154.94 93.98) (end 154.12001 93.98) (width 0.25) (layer B.Cu) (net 3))
 (via (at 135.89 109.22) (size 0.8) (drill 0.4) (layers F.Cu B.Cu) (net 3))
 (segment (start 125.334998 109.22) (end 135.89 109.22) (width 0.25) (layer F.Cu) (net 3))
 (segment (start 122.064999 105.950001) (end 125.334998 109.22) (width 0.25) (layer F.Cu) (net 3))
 (segment (start 122.064999 103.014999) (end 122.064999 105.950001) (width 0.25) (layer F.Cu) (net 3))
 (segment (start 120.65 101.6) (end 122.064999 103.014999) (width 0.25) (layer F.Cu) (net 3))
 (segment (start 156.065001 95.105001) (end 154.94 93.98) (width 0.25) (layer B.Cu) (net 3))
 (segment (start 155.480001 97.645001) (end 156.065001 97.060001) (width 0.25) (layer B.Cu) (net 3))
 (segment (start 154.399999 97.645001) (end 155.480001 97.645001) (width 0.25) (layer B.Cu) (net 3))
 (segment (start 153.67 98.375) (end 154.399999 97.645001) (width 0.25) (layer B.Cu) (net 3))
 (segment (start 153.67 100.725002) (end 153.67 98.375) (width 0.25) (layer B.Cu) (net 3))
 (segment (start 156.065001 97.060001) (end 156.065001 95.105001) (width 0.25) (layer B.Cu) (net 3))
 (segment (start 151.670001 102.725001) (end 153.67 100.725002) (width 0.25) (layer B.Cu) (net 3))
 (segment (start 146.391997 102.725001) (end 151.670001 102.725001) (width 0.25) (layer B.Cu) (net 3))
 (segment (start 139.896998 109.22) (end 146.391997 102.725001) (width 0.25) (layer B.Cu) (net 3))
 (segment (start 135.89 109.22) (end 139.896998 109.22) (width 0.25) (layer B.Cu) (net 3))
 (via (at 149.86 96.52) (size 0.8) (drill 0.4) (layers F.Cu B.Cu) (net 24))
 (segment (start 154.94 96.52) (end 149.86 96.52) (width 0.25) (layer F.Cu) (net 24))
 (segment (start 133.35 96.52) (end 123.19 86.36) (width 0.25) (layer B.Cu) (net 24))
 (segment (start 149.86 96.52) (end 133.35 96.52) (width 0.25) (layer B.Cu) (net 24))
 (segment (start 150.056998 97.79) (end 148.59 97.79) (width 0.25) (layer F.Cu) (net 1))
 (segment (start 151.326998 99.06) (end 150.056998 97.79) (width 0.25) (layer F.Cu) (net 1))
 (via (at 148.59 97.79) (size 0.8) (drill 0.4) (layers F.Cu B.Cu) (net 1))
 (segment (start 154.94 99.06) (end 151.326998 99.06) (width 0.25) (layer F.Cu) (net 1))
 (segment (start 147.864999 97.064999) (end 122.645001 97.064999) (width 0.25) (layer B.Cu) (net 1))
 (segment (start 122.645001 97.064999) (end 118.11 101.6) (width 0.25) (layer B.Cu) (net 1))
 (segment (start 148.59 97.79) (end 147.864999 97.064999) (width 0.25) (layer B.Cu) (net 1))
 (via (at 133.35 93.98) (size 0.8) (drill 0.4) (layers F.Cu B.Cu) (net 16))
 (segment (start 133.35 86.36) (end 133.35 93.98) (width 0.25) (layer B.Cu) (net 16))
 (via (at 147.32 103.450001) (size 0.8) (drill 0.4) (layers F.Cu B.Cu) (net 16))
 (segment (start 147.284998 103.414999) (end 147.32 103.450001) (width 0.25) (layer F.Cu) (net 16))
 (segment (start 144.924999 102.140001) (end 146.199997 103.414999) (width 0.25) (layer F.Cu) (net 16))
 (segment (start 146.199997 103.414999) (end 147.284998 103.414999) (width 0.25) (layer F.Cu) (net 16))
 (segment (start 144.924999 101.059999) (end 144.924999 102.140001) (width 0.25) (layer F.Cu) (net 16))
 (segment (start 136.231997 100.474999) (end 144.339999 100.474999) (width 0.25) (layer F.Cu) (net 16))
 (segment (start 144.339999 100.474999) (end 144.924999 101.059999) (width 0.25) (layer F.Cu) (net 16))
 (segment (start 133.35 97.593002) (end 136.231997 100.474999) (width 0.25) (layer F.Cu) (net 16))
 (segment (start 133.35 93.98) (end 133.35 97.593002) (width 0.25) (layer F.Cu) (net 16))
 (segment (start 153.089999 103.450001) (end 154.94 101.6) (width 0.25) (layer B.Cu) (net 16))
 (segment (start 147.32 103.450001) (end 153.089999 103.450001) (width 0.25) (layer B.Cu) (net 16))
 (segment (start 129.684999 83.279999) (end 126.604998 86.36) (width 0.25) (layer F.Cu) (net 22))
 (segment (start 129.684999 82.009999) (end 129.684999 83.279999) (width 0.25) (layer F.Cu) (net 22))
 (segment (start 130.269999 81.424999) (end 129.684999 82.009999) (width 0.25) (layer F.Cu) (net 22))
 (segment (start 126.604998 86.36) (end 125.73 86.36) (width 0.25) (layer F.Cu) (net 22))
 (segment (start 141.510001 81.424999) (end 130.269999 81.424999) (width 0.25) (layer F.Cu) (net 22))
 (segment (start 142.095001 82.009999) (end 141.510001 81.424999) (width 0.25) (layer F.Cu) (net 22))
 (segment (start 142.095001 87.036405) (end 142.095001 82.009999) (width 0.25) (layer F.Cu) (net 22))
 (segment (start 142.833595 87.774999) (end 142.095001 87.036405) (width 0.25) (layer F.Cu) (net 22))
 (segment (start 161.434999 87.774999) (end 142.833595 87.774999) (width 0.25) (layer F.Cu) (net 22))
 (segment (start 162.56 88.9) (end 161.434999 87.774999) (width 0.25) (layer F.Cu) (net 22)))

